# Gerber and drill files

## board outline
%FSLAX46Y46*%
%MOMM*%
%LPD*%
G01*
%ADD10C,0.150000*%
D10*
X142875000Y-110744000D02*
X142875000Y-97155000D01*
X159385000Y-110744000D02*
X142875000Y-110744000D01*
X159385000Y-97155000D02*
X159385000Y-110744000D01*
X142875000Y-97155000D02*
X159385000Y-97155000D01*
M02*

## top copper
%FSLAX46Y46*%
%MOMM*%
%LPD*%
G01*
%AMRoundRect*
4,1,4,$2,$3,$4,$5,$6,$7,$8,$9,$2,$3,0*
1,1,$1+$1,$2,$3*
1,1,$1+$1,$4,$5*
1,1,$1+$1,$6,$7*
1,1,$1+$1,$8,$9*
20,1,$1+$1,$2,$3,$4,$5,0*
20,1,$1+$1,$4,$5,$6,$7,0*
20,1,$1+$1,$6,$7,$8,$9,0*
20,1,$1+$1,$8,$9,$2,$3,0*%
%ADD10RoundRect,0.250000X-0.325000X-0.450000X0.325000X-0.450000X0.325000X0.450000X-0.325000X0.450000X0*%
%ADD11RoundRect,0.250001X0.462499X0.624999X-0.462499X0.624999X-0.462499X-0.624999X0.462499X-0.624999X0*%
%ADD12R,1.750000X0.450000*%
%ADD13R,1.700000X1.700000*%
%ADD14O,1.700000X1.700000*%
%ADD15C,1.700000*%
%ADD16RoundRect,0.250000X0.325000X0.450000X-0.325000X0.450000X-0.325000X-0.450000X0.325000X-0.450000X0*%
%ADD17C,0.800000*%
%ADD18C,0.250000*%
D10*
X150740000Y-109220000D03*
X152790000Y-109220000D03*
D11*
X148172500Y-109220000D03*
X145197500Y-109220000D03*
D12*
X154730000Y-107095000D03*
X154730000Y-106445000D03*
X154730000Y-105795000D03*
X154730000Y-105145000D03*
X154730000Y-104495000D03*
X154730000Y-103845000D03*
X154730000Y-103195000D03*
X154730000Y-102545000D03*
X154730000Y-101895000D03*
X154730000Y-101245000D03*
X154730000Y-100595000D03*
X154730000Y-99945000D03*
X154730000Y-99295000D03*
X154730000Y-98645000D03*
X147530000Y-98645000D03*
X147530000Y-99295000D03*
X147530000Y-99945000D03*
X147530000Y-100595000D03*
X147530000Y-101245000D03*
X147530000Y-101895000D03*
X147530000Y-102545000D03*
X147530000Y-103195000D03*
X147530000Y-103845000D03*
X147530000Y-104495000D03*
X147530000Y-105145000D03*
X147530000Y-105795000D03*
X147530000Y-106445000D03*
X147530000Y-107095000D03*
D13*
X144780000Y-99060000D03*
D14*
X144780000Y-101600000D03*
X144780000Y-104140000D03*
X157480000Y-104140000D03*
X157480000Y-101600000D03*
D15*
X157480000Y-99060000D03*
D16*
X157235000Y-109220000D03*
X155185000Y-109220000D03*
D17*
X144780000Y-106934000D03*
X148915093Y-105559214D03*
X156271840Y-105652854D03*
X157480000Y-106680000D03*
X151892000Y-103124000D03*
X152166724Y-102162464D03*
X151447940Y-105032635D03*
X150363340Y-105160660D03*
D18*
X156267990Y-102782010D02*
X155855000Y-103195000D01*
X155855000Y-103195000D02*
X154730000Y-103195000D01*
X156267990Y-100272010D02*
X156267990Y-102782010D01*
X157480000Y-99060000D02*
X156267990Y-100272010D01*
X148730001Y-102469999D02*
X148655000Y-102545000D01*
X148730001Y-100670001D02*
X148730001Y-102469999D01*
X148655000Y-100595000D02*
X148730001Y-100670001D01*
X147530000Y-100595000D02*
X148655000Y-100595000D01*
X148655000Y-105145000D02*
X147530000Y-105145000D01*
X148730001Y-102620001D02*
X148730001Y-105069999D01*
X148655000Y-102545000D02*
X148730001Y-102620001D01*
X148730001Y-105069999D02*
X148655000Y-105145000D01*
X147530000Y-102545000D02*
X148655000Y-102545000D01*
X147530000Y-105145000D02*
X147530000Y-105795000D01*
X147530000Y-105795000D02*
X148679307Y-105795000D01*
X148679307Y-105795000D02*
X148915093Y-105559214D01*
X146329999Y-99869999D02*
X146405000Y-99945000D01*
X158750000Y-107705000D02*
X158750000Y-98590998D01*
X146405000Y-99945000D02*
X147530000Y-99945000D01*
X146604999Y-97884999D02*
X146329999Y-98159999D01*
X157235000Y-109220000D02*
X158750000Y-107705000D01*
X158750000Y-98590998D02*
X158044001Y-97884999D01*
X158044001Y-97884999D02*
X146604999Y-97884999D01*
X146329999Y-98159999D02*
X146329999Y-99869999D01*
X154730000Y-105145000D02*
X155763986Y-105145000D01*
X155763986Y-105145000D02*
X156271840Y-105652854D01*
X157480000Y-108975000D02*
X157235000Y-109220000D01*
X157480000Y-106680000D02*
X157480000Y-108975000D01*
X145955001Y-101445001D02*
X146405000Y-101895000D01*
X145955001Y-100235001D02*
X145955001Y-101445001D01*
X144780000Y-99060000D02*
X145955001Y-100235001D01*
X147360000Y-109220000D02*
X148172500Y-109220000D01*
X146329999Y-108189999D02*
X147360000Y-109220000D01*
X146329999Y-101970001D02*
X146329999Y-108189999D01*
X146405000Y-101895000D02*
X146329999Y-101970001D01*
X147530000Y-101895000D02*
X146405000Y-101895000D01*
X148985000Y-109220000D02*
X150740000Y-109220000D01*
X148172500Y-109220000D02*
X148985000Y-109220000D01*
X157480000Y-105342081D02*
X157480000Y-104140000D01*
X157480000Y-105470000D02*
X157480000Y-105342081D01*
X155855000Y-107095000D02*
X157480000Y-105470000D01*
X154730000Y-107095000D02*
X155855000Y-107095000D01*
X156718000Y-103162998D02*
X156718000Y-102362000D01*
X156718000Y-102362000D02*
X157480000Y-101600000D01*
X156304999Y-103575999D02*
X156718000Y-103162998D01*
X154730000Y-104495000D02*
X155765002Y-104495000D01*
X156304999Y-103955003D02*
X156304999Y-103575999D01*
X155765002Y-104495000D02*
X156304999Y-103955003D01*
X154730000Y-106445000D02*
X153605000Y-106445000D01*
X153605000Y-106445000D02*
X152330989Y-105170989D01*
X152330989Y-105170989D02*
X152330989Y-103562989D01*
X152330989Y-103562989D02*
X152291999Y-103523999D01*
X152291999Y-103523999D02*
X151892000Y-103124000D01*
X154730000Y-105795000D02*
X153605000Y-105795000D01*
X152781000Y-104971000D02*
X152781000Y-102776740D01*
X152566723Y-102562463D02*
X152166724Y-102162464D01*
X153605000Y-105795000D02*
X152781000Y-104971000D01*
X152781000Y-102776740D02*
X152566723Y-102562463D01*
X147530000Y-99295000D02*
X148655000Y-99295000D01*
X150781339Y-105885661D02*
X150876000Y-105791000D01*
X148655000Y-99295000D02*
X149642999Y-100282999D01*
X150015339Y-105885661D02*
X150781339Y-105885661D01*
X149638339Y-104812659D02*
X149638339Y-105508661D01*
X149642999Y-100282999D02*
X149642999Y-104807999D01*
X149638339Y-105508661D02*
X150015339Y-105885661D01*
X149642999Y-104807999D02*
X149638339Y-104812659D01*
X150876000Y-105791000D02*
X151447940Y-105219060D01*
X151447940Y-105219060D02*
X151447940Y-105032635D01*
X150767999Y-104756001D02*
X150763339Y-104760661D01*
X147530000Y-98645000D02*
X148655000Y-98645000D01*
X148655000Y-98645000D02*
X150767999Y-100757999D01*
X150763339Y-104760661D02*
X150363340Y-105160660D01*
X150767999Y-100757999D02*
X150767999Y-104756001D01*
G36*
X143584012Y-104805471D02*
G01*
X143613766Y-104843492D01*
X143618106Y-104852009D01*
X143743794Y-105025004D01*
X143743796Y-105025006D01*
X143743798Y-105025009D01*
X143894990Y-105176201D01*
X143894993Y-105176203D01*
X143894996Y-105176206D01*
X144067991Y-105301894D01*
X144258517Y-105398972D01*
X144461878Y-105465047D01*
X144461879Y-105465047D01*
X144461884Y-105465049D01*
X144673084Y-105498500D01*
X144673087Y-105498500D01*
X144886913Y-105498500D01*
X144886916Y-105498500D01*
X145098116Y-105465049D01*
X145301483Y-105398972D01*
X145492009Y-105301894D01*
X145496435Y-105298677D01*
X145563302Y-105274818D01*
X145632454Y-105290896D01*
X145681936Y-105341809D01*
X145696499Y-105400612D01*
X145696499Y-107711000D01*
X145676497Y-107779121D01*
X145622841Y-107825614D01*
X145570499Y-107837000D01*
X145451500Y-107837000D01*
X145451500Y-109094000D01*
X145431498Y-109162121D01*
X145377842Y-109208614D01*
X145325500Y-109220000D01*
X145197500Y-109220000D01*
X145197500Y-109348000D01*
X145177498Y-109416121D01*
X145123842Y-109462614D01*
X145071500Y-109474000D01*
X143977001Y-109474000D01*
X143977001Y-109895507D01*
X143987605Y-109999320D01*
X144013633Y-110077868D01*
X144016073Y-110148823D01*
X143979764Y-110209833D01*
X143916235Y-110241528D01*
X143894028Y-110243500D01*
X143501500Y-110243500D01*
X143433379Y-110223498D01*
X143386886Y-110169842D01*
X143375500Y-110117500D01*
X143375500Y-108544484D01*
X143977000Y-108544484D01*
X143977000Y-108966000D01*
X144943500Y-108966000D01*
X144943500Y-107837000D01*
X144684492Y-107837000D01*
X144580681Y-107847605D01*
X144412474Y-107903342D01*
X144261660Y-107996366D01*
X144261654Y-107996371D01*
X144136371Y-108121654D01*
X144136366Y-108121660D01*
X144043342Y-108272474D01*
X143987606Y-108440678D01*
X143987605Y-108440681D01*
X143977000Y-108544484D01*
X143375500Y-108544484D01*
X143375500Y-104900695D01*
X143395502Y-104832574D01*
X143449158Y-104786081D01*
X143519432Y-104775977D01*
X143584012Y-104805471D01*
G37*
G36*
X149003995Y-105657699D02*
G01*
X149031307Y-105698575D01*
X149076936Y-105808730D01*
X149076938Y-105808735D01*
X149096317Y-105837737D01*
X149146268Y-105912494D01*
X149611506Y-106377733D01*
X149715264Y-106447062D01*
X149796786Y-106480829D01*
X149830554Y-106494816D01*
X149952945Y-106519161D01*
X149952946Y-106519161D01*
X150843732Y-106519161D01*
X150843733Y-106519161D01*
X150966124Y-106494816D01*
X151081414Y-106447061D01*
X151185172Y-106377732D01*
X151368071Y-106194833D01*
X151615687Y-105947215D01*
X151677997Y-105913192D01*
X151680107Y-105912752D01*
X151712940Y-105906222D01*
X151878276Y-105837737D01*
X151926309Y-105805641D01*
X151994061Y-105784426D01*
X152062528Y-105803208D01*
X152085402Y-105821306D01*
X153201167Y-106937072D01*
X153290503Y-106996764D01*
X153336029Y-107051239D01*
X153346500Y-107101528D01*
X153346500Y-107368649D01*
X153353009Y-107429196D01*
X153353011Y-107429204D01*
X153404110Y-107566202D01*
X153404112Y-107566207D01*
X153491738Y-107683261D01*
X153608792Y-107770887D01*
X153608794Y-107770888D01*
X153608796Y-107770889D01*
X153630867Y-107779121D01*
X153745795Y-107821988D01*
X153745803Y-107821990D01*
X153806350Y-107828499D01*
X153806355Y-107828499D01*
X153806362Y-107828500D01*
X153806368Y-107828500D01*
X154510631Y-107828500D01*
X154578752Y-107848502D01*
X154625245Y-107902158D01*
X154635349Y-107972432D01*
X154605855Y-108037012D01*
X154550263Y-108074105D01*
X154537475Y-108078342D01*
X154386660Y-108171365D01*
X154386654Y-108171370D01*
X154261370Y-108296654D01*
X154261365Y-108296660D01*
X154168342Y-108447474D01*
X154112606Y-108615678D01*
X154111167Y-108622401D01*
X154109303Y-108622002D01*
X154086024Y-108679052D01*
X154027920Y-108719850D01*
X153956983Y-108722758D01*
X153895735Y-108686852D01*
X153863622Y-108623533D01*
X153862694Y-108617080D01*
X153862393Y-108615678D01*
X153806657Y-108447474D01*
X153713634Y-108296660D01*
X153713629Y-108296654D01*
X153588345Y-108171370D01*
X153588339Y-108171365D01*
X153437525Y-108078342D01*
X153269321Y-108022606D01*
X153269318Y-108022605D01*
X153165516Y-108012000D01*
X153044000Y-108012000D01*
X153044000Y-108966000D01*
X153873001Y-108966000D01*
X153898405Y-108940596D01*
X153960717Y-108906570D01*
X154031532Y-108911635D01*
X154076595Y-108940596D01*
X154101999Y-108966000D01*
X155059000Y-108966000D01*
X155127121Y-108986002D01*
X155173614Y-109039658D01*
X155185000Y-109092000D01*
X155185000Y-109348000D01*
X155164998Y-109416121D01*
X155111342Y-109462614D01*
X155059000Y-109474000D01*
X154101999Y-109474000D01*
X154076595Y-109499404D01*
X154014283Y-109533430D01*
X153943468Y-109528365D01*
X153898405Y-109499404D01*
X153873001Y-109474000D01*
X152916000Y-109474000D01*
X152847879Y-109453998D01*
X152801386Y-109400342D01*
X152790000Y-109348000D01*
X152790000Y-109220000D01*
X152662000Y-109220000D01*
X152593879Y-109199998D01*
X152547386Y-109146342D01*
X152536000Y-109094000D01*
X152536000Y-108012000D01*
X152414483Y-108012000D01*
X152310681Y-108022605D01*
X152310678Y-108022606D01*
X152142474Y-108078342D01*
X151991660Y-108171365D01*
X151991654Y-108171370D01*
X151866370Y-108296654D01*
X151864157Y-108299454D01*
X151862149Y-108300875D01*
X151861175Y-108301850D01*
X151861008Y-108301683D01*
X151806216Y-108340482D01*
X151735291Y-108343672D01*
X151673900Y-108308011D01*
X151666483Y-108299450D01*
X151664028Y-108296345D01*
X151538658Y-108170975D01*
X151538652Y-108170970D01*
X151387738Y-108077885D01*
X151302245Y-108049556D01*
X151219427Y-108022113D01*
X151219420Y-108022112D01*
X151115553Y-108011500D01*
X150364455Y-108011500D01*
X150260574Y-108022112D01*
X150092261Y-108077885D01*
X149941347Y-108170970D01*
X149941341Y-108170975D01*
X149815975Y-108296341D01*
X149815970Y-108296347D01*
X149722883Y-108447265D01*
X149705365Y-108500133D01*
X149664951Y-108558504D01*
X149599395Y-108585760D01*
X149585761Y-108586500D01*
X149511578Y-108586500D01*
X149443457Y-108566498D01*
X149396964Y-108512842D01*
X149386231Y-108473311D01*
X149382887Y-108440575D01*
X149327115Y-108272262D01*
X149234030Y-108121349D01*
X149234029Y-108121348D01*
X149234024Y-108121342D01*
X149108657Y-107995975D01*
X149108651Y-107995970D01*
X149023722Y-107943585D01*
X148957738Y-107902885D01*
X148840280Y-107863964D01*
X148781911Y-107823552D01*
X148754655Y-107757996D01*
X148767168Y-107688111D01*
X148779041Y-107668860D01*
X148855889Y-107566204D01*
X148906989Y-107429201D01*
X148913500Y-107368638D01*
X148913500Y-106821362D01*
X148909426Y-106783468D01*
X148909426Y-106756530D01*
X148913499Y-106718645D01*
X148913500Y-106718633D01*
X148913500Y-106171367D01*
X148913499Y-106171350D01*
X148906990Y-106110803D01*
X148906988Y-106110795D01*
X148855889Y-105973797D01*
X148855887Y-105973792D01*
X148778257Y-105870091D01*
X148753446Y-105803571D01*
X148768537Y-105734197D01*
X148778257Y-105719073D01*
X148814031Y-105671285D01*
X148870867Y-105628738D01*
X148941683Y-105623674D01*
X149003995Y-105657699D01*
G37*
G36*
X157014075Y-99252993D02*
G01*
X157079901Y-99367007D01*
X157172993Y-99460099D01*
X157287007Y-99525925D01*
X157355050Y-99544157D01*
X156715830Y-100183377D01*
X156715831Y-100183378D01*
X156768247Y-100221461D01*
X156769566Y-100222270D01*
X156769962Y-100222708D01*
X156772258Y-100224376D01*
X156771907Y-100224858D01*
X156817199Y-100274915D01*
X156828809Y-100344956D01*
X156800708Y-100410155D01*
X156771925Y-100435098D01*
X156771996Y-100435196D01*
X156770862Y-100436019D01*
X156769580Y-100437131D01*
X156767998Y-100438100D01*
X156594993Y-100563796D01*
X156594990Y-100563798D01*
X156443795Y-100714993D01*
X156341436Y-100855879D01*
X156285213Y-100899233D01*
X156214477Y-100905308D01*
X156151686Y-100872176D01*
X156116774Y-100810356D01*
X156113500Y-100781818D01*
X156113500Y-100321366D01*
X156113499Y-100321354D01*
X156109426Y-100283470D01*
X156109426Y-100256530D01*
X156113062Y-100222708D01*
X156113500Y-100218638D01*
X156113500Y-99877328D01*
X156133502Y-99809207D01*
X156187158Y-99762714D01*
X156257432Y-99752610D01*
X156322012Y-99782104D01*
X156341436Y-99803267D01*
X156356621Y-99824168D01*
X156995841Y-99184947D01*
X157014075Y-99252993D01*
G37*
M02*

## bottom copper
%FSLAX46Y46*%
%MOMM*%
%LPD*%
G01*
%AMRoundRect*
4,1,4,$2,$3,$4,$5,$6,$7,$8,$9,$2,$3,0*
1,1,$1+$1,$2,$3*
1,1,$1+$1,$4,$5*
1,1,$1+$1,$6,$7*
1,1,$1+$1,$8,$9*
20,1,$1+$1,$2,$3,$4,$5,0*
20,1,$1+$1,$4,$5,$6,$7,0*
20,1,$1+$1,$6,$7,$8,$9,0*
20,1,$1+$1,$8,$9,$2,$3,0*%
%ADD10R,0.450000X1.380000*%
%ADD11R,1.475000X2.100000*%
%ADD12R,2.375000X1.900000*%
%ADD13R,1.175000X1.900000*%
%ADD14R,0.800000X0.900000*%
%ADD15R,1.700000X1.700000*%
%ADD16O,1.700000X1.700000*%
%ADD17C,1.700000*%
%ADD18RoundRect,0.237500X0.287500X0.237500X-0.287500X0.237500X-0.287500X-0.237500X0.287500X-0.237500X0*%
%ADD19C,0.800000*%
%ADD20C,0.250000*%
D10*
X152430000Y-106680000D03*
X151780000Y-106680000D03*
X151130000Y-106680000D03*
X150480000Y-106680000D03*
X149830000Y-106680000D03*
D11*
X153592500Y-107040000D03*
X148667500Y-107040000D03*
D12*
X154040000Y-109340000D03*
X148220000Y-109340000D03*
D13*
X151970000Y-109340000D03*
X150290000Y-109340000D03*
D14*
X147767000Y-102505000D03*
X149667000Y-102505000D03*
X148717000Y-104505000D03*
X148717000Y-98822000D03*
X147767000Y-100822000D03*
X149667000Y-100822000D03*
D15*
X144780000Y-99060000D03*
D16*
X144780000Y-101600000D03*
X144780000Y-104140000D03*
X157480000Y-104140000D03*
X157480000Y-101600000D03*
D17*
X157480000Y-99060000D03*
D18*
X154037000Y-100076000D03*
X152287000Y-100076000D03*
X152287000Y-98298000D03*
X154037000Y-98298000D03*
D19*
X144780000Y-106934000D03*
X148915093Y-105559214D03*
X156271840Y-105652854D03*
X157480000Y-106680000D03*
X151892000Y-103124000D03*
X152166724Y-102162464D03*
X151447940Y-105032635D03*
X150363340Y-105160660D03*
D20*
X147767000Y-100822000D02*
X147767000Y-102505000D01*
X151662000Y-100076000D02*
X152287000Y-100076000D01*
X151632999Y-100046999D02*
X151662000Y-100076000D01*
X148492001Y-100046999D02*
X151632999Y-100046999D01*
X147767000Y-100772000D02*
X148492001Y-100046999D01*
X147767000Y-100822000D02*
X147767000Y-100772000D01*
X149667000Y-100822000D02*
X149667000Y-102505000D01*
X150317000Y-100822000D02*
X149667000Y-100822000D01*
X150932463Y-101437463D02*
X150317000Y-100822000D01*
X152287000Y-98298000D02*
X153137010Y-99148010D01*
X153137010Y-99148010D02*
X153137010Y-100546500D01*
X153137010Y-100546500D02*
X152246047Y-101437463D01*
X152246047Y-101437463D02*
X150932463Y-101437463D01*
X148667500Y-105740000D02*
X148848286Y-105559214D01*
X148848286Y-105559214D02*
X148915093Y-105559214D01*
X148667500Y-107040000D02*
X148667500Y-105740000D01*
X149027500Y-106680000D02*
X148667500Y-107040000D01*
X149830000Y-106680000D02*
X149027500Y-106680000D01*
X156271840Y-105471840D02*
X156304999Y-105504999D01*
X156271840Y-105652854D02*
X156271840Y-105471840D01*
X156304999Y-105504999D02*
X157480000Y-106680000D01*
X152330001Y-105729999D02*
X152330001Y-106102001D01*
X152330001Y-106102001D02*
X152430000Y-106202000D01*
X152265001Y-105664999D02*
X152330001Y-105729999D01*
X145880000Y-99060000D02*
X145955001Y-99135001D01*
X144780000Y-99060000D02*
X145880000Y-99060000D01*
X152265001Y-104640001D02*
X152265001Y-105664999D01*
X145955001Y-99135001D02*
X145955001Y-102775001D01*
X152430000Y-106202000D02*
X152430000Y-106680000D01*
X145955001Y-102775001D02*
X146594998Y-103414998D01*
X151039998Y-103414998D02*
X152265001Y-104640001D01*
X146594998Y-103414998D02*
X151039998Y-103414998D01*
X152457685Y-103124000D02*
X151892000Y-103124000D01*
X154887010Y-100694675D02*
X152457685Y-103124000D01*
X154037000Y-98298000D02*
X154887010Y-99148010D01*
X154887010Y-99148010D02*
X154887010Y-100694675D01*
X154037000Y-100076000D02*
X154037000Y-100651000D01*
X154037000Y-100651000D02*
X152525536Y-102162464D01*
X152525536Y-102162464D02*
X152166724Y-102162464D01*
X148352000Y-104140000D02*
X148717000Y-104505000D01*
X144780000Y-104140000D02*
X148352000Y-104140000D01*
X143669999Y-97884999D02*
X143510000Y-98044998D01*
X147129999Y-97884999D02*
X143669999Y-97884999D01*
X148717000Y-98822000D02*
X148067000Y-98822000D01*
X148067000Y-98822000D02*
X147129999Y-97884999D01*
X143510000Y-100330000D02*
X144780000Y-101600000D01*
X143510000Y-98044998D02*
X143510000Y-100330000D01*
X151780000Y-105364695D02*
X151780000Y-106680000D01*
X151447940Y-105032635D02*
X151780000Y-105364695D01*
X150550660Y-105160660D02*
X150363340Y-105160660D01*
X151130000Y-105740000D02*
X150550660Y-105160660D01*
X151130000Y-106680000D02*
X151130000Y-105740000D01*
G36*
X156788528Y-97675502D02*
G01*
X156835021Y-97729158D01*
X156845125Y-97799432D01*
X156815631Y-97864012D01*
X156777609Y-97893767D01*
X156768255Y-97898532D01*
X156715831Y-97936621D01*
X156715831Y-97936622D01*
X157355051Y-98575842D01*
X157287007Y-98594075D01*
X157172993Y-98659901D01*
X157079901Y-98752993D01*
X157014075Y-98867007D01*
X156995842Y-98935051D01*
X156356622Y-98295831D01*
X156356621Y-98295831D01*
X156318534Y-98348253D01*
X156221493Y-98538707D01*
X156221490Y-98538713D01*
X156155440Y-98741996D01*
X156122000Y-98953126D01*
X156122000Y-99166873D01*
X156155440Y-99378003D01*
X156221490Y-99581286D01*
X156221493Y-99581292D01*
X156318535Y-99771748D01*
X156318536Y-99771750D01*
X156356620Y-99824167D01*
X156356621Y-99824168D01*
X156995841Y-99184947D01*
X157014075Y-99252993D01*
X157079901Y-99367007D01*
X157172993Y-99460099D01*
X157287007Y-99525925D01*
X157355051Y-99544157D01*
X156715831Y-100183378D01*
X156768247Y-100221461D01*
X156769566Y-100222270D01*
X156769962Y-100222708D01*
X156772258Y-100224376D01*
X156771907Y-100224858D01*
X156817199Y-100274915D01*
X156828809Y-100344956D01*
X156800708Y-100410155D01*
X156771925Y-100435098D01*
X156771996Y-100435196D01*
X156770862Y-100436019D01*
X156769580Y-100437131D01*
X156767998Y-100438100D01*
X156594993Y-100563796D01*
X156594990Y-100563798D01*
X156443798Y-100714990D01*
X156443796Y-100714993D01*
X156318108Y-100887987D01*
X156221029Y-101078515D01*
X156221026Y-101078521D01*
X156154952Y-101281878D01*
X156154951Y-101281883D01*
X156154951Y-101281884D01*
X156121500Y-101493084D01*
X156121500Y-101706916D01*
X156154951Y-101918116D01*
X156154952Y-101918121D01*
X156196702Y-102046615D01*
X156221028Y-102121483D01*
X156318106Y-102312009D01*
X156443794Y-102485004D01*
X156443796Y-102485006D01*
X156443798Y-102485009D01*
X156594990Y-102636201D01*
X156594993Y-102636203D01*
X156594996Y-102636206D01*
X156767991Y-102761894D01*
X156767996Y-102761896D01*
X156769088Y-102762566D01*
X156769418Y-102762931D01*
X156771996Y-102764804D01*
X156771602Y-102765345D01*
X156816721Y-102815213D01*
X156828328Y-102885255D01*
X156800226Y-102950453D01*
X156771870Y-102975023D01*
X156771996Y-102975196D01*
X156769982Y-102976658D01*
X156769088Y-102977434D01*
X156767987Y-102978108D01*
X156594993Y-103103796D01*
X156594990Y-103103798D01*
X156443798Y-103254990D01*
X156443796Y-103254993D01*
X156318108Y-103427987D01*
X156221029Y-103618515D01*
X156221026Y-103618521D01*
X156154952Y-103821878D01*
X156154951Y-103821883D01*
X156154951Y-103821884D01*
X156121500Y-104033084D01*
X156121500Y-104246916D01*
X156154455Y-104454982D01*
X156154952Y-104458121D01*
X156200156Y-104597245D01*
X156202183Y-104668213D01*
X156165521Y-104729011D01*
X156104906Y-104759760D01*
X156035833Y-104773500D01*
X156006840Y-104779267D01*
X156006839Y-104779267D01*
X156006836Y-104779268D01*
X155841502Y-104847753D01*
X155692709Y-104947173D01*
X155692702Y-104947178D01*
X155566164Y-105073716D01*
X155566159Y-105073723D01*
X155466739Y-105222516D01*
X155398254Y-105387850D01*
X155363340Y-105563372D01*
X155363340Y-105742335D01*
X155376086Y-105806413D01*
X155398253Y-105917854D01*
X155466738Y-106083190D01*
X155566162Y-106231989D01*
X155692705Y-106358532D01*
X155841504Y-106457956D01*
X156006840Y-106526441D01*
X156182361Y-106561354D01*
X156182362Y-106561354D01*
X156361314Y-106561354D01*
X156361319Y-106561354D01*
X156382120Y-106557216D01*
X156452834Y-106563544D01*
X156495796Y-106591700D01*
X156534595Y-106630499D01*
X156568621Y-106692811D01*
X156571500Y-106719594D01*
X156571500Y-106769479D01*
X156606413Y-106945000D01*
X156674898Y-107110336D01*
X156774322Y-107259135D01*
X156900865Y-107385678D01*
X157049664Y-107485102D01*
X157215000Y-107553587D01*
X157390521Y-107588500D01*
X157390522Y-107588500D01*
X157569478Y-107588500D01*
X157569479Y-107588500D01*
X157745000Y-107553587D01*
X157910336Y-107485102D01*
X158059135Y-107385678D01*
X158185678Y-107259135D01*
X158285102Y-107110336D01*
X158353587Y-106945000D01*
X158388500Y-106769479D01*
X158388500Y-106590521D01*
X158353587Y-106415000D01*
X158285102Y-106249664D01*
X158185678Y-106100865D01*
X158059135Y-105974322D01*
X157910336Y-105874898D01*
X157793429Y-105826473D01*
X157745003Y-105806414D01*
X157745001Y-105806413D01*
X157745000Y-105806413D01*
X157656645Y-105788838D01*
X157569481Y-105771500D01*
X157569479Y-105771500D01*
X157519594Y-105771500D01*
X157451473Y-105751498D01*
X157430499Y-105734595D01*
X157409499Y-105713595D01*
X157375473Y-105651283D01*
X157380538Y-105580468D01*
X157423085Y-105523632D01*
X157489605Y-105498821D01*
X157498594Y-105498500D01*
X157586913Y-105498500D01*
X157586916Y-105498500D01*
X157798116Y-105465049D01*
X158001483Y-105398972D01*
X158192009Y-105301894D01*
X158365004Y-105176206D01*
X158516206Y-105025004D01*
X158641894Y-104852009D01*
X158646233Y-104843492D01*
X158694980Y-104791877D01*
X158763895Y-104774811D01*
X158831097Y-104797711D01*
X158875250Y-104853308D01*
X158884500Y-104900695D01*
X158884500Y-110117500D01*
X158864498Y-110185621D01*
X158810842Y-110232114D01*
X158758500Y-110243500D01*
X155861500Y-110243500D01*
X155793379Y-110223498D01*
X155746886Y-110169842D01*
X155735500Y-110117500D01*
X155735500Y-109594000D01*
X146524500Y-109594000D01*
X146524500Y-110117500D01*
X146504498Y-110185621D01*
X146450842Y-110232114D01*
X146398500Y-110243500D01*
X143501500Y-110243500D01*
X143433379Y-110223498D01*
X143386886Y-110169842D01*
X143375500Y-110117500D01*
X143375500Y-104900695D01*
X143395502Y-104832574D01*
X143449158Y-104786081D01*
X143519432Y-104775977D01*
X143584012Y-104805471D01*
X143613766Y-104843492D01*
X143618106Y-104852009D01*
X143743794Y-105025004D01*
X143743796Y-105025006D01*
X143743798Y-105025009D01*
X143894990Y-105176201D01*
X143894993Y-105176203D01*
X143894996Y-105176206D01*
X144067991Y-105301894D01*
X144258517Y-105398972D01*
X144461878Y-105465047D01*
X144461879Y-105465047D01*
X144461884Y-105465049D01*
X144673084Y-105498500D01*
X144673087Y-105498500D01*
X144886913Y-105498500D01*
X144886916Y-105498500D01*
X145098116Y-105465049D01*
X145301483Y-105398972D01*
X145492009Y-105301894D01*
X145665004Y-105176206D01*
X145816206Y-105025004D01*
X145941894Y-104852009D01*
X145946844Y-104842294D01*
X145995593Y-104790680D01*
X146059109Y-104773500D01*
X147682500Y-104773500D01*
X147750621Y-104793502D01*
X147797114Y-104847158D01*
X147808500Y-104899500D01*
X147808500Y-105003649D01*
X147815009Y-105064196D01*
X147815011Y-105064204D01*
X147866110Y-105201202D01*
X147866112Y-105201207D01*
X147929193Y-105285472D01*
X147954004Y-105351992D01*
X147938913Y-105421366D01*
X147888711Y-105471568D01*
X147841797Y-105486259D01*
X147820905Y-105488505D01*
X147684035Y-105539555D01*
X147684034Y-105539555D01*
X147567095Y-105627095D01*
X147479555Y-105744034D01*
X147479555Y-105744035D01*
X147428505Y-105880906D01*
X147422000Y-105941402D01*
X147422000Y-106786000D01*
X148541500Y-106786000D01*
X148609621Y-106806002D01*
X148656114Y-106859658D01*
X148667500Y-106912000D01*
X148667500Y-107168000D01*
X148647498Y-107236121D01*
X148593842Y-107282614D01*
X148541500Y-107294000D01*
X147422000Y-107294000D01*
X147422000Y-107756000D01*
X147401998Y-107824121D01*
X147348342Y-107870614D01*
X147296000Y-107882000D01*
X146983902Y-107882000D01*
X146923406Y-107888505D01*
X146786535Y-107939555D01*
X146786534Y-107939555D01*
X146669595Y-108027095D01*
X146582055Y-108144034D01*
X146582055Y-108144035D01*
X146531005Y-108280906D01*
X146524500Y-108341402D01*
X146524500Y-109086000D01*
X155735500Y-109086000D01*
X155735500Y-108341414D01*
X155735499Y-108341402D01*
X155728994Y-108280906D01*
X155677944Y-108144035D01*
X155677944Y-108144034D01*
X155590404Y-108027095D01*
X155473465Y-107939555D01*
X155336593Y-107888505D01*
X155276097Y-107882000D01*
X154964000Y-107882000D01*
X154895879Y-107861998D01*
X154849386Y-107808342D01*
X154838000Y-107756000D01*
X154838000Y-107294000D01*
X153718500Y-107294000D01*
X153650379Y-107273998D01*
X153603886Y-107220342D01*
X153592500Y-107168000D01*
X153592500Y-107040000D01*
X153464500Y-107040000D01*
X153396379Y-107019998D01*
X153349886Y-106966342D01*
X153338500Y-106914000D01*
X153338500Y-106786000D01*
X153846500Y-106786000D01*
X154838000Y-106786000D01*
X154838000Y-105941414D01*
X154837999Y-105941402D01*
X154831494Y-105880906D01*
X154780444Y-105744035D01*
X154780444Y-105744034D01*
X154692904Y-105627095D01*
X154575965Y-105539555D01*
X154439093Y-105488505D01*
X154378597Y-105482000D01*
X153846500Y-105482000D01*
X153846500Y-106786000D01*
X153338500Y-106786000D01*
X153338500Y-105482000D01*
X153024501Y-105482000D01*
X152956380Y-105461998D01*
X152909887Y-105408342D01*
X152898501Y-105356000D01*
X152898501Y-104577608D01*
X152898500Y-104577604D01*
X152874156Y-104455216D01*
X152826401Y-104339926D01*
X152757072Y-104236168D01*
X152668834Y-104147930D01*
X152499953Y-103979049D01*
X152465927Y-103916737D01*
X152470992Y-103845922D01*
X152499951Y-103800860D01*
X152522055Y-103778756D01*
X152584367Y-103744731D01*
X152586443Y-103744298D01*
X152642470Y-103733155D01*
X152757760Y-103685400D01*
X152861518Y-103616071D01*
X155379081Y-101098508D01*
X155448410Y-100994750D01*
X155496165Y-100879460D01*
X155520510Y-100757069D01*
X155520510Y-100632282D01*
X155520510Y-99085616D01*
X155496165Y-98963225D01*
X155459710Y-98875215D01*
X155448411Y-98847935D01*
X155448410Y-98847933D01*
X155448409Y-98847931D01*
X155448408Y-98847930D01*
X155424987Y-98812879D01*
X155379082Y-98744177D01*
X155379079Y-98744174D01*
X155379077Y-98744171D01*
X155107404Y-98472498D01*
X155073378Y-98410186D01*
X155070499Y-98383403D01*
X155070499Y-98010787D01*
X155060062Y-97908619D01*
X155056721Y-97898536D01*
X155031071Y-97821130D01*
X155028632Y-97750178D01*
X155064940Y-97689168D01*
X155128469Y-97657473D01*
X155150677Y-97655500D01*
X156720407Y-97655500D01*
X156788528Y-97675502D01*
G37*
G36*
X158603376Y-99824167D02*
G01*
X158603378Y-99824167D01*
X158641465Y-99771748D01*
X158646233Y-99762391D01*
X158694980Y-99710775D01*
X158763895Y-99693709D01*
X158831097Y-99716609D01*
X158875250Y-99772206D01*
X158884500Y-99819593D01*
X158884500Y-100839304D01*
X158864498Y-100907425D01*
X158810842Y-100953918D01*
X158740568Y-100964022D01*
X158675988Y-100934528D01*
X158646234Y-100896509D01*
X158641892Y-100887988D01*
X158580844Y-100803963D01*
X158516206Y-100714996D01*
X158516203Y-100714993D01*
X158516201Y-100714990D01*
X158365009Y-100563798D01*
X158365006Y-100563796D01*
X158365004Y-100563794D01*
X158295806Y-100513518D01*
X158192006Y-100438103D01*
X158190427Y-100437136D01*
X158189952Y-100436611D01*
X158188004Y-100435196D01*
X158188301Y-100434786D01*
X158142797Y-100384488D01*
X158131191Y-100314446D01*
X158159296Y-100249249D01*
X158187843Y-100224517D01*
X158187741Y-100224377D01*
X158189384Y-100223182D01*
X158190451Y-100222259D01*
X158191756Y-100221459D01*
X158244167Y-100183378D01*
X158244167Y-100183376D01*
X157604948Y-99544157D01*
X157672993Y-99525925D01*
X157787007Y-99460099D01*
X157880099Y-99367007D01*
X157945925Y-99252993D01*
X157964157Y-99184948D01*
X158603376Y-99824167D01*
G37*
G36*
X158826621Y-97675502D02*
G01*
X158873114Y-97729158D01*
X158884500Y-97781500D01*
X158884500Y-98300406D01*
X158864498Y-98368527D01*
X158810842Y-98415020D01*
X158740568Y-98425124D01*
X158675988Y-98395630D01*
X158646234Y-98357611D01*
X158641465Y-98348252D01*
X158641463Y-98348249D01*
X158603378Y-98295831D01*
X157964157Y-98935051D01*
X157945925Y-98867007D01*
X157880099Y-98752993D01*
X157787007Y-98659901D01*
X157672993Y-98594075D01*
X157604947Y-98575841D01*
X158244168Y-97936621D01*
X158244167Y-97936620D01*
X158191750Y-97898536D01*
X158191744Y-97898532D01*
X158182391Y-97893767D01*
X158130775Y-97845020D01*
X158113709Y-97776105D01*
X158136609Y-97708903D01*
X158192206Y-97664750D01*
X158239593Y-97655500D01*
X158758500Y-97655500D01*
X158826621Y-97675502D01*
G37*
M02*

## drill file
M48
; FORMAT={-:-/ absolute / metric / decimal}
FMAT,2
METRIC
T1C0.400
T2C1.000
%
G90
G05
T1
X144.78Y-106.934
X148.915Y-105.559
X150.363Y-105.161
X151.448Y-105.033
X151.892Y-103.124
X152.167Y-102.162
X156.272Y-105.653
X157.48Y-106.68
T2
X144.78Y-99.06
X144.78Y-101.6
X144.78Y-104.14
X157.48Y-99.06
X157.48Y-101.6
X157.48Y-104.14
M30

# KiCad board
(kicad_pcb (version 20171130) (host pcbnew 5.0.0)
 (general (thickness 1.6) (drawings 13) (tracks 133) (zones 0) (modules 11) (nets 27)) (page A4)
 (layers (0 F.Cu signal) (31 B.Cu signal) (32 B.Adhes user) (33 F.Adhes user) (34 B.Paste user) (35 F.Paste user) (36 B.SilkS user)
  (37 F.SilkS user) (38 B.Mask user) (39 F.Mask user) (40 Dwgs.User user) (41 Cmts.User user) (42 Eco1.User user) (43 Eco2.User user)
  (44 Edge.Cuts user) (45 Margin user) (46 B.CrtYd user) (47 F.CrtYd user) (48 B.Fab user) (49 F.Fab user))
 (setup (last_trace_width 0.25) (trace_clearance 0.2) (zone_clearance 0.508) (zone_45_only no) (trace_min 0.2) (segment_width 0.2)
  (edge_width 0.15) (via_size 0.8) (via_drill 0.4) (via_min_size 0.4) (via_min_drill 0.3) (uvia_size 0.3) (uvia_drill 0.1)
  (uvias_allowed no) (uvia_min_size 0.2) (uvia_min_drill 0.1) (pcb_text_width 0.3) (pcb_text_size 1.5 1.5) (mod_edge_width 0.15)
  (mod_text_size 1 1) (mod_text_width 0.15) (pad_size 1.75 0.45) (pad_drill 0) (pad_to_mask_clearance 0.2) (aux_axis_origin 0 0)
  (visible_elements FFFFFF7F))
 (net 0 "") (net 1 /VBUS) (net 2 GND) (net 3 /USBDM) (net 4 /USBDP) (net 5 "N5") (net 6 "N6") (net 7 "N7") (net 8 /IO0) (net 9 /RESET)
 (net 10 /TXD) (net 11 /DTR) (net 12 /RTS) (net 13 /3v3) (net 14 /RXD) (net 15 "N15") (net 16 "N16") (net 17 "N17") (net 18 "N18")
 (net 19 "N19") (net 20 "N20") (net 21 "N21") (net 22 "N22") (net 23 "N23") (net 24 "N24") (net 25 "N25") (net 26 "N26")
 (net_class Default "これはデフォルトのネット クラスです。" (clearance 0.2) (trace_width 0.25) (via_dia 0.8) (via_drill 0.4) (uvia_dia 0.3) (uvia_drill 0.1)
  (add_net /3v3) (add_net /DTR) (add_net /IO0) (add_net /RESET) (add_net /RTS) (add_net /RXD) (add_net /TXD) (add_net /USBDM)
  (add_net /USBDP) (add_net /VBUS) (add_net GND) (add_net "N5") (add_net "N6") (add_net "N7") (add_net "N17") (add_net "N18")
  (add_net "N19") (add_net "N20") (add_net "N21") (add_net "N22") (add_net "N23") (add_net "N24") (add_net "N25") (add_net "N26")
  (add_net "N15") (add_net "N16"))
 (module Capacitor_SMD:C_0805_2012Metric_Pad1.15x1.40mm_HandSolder (layer F.Cu) (at 151.765 109.22)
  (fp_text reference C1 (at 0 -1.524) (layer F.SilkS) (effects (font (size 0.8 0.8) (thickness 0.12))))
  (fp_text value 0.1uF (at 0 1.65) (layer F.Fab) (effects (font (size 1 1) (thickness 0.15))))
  (pad 1 smd roundrect (at -1.025 0) (size 1.15 1.4) (layers F.Cu F.Paste F.Mask) (roundrect_rratio 0.217391) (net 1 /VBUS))
  (pad 2 smd roundrect (at 1.025 0) (size 1.15 1.4) (layers F.Cu F.Paste F.Mask) (roundrect_rratio 0.217391) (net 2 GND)))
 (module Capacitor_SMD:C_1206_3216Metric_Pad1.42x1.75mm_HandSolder (layer F.Cu) (at 146.685 109.22 180)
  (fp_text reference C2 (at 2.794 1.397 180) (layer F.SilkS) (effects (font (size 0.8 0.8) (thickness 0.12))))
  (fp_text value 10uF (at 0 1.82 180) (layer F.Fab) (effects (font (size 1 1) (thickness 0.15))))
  (pad 1 smd roundrect (at -1.4875 0 180) (size 1.425 1.75) (layers F.Cu F.Paste F.Mask) (roundrect_rratio 0.175439) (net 1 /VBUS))
  (pad 2 smd roundrect (at 1.4875 0 180) (size 1.425 1.75) (layers F.Cu F.Paste F.Mask) (roundrect_rratio 0.175439) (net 2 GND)))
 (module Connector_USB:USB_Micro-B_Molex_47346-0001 (layer B.Cu) (at 151.13 108.14 180)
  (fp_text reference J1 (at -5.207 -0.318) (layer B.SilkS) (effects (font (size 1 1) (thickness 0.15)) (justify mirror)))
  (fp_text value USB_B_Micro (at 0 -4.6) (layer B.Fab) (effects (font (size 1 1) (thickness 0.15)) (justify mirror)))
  (pad 1 smd rect (at -1.3 1.46 180) (size 0.45 1.38) (layers B.Cu B.Paste B.Mask) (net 1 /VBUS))
  (pad 2 smd rect (at -0.65 1.46 180) (size 0.45 1.38) (layers B.Cu B.Paste B.Mask) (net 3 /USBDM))
  (pad 3 smd rect (at 0 1.46 180) (size 0.45 1.38) (layers B.Cu B.Paste B.Mask) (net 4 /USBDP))
  (pad 4 smd rect (at 0.65 1.46 180) (size 0.45 1.38) (layers B.Cu B.Paste B.Mask) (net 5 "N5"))
  (pad 5 smd rect (at 1.3 1.46 180) (size 0.45 1.38) (layers B.Cu B.Paste B.Mask) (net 2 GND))
  (pad 6 smd rect (at -2.4625 1.1 180) (size 1.475 2.1) (layers B.Cu B.Paste B.Mask) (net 2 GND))
  (pad 6 smd rect (at 2.4625 1.1 180) (size 1.475 2.1) (layers B.Cu B.Paste B.Mask) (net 2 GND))
  (pad 6 smd rect (at -2.91 -1.2 180) (size 2.375 1.9) (layers B.Cu B.Paste B.Mask) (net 2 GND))
  (pad 6 smd rect (at 2.91 -1.2 180) (size 2.375 1.9) (layers B.Cu B.Paste B.Mask) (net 2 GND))
  (pad 6 smd rect (at -0.84 -1.2 180) (size 1.175 1.9) (layers B.Cu B.Paste B.Mask) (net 2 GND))
  (pad 6 smd rect (at 0.84 -1.2 180) (size 1.175 1.9) (layers B.Cu B.Paste B.Mask) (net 2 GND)))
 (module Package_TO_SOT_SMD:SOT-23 (layer B.Cu) (at 148.717 103.505 270)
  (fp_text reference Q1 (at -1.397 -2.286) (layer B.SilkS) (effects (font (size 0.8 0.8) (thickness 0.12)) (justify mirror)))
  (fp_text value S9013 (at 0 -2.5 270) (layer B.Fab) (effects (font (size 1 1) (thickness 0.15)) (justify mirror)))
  (pad 1 smd rect (at -1 0.95 270) (size 0.9 0.8) (layers B.Cu B.Paste B.Mask) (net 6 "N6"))
  (pad 2 smd rect (at -1 -0.95 270) (size 0.9 0.8) (layers B.Cu B.Paste B.Mask) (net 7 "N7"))
  (pad 3 smd rect (at 1 0 270) (size 0.9 0.8) (layers B.Cu B.Paste B.Mask) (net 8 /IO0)))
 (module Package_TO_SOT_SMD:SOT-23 (layer B.Cu) (at 148.717 99.822 90)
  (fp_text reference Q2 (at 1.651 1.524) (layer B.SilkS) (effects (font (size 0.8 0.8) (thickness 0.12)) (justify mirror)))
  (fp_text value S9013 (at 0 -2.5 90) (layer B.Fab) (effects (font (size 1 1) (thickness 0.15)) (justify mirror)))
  (pad 3 smd rect (at 1 0 90) (size 0.9 0.8) (layers B.Cu B.Paste B.Mask) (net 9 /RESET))
  (pad 2 smd rect (at -1 -0.95 90) (size 0.9 0.8) (layers B.Cu B.Paste B.Mask) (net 6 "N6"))
  (pad 1 smd rect (at -1 0.95 90) (size 0.9 0.8) (layers B.Cu B.Paste B.Mask) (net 7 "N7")))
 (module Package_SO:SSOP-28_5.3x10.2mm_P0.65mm (layer F.Cu) (at 151.13 102.87 180)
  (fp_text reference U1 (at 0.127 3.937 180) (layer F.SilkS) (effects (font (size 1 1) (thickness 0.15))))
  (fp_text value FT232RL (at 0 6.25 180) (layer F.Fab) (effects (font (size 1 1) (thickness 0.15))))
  (pad 1 smd rect (at -3.6 -4.225 180) (size 1.75 0.45) (layers F.Cu F.Paste F.Mask) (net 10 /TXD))
  (pad 2 smd rect (at -3.6 -3.575 180) (size 1.75 0.45) (layers F.Cu F.Paste F.Mask) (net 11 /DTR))
  (pad 3 smd rect (at -3.6 -2.925 180) (size 1.75 0.45) (layers F.Cu F.Paste F.Mask) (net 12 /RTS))
  (pad 4 smd rect (at -3.6 -2.275 180) (size 1.75 0.45) (layers F.Cu F.Paste F.Mask) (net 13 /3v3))
  (pad 5 smd rect (at -3.6 -1.625 180) (size 1.75 0.45) (layers F.Cu F.Paste F.Mask) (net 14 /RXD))
  (pad 6 smd rect (at -3.6 -0.975 180) (size 1.75 0.45) (layers F.Cu F.Paste F.Mask) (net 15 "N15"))
  (pad 7 smd rect (at -3.6 -0.325 180) (size 1.75 0.45) (layers F.Cu F.Paste F.Mask) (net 2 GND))
  (pad 8 smd rect (at -3.6 0.325 180) (size 1.75 0.45) (layers F.Cu F.Paste F.Mask))
  (pad 9 smd rect (at -3.6 0.975 180) (size 1.75 0.45) (layers F.Cu F.Paste F.Mask) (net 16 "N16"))
  (pad 10 smd rect (at -3.6 1.625 180) (size 1.75 0.45) (layers F.Cu F.Paste F.Mask) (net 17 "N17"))
  (pad 11 smd rect (at -3.6 2.275 180) (size 1.75 0.45) (layers F.Cu F.Paste F.Mask) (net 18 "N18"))
  (pad 12 smd rect (at -3.6 2.925 180) (size 1.75 0.45) (layers F.Cu F.Paste F.Mask) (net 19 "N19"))
  (pad 13 smd rect (at -3.6 3.575 180) (size 1.75 0.45) (layers F.Cu F.Paste F.Mask) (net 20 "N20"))
  (pad 14 smd rect (at -3.6 4.225 180) (size 1.75 0.45) (layers F.Cu F.Paste F.Mask) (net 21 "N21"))
  (pad 15 smd rect (at 3.6 4.225 180) (size 1.75 0.45) (layers F.Cu F.Paste F.Mask) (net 4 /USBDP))
  (pad 16 smd rect (at 3.6 3.575 180) (size 1.75 0.45) (layers F.Cu F.Paste F.Mask) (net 3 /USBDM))
  (pad 17 smd rect (at 3.6 2.925 180) (size 1.75 0.45) (layers F.Cu F.Paste F.Mask) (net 13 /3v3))
  (pad 18 smd rect (at 3.6 2.275 180) (size 1.75 0.45) (layers F.Cu F.Paste F.Mask) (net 2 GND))
  (pad 19 smd rect (at 3.6 1.625 180) (size 1.75 0.45) (layers F.Cu F.Paste F.Mask) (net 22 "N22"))
  (pad 20 smd rect (at 3.6 0.975 180) (size 1.75 0.45) (layers F.Cu F.Paste F.Mask) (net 1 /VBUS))
  (pad 21 smd rect (at 3.6 0.325 180) (size 1.75 0.45) (layers F.Cu F.Paste F.Mask) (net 2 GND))
  (pad 22 smd rect (at 3.6 -0.325 180) (size 1.75 0.45) (layers F.Cu F.Paste F.Mask) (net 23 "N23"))
  (pad 23 smd rect (at 3.6 -0.975 180) (size 1.75 0.45) (layers F.Cu F.Paste F.Mask) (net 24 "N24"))
  (pad 24 smd rect (at 3.6 -1.625 180) (size 1.75 0.45) (layers F.Cu F.Paste F.Mask))
  (pad 25 smd rect (at 3.6 -2.275 180) (size 1.75 0.45) (layers F.Cu F.Paste F.Mask) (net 2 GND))
  (pad 26 smd rect (at 3.6 -2.925 180) (size 1.75 0.45) (layers F.Cu F.Paste F.Mask) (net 2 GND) (zone_connect 2))
  (pad 27 smd rect (at 3.6 -3.575 180) (size 1.75 0.45) (layers F.Cu F.Paste F.Mask) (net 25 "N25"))
  (pad 28 smd rect (at 3.6 -4.225 180) (size 1.75 0.45) (layers F.Cu F.Paste F.Mask) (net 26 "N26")))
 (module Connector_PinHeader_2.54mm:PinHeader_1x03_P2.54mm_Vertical (layer B.Cu) (at 144.78 99.06 180)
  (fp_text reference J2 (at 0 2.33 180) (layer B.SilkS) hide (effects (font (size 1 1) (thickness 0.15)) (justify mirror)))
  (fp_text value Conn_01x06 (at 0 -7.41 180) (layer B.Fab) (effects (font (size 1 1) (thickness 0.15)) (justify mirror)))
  (pad 1 thru_hole rect (at 0 0 180) (size 1.7 1.7) (drill 1) (layers *.Cu *.Mask) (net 1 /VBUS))
  (pad 2 thru_hole oval (at 0 -2.54 180) (size 1.7 1.7) (drill 1) (layers *.Cu *.Mask) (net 9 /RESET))
  (pad 3 thru_hole oval (at 0 -5.08 180) (size 1.7 1.7) (drill 1) (layers *.Cu *.Mask) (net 8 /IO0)))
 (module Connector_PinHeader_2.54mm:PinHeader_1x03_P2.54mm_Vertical (layer B.Cu) (at 157.48 99.06 180)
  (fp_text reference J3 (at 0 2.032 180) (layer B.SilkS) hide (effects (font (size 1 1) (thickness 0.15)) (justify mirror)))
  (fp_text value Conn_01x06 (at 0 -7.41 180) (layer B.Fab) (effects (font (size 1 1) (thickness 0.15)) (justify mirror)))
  (pad 3 thru_hole oval (at 0 -5.08 180) (size 1.7 1.7) (drill 1) (layers *.Cu *.Mask) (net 10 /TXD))
  (pad 2 thru_hole oval (at 0 -2.54 180) (size 1.7 1.7) (drill 1) (layers *.Cu *.Mask) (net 14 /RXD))
  (pad 1 thru_hole circle (at 0 0 180) (size 1.7 1.7) (drill 1) (layers *.Cu *.Mask) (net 2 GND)))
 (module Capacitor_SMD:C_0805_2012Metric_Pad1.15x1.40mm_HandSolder (layer F.Cu) (at 156.21 109.22 180)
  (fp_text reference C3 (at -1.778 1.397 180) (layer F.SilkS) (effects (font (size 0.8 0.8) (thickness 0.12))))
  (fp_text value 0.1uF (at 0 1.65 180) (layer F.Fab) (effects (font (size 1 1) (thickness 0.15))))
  (pad 1 smd roundrect (at -1.025 0 180) (size 1.15 1.4) (layers F.Cu F.Paste F.Mask) (roundrect_rratio 0.217391) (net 13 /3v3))
  (pad 2 smd roundrect (at 1.025 0 180) (size 1.15 1.4) (layers F.Cu F.Paste F.Mask) (roundrect_rratio 0.217391) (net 2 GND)))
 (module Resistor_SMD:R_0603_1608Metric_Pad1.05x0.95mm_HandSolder (layer B.Cu) (at 153.162 100.076 180)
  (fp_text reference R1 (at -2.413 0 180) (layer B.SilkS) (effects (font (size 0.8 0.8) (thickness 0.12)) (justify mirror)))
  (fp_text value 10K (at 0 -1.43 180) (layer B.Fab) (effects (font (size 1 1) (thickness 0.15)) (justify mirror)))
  (pad 1 smd roundrect (at -0.875 0 180) (size 1.05 0.95) (layers B.Cu B.Paste B.Mask) (roundrect_rratio 0.25) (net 12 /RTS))
  (pad 2 smd roundrect (at 0.875 0 180) (size 1.05 0.95) (layers B.Cu B.Paste B.Mask) (roundrect_rratio 0.25) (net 6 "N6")))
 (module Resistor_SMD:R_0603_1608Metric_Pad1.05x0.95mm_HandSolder (layer B.Cu) (at 153.162 98.298 180)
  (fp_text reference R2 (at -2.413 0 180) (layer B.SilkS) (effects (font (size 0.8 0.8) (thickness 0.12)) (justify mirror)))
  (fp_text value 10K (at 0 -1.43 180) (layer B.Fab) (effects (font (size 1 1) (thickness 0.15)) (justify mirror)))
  (pad 2 smd roundrect (at 0.875 0 180) (size 1.05 0.95) (layers B.Cu B.Paste B.Mask) (roundrect_rratio 0.25) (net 7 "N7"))
  (pad 1 smd roundrect (at -0.875 0 180) (size 1.05 0.95) (layers B.Cu B.Paste B.Mask) (roundrect_rratio 0.25) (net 11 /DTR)))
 (gr_line (start 142.875 110.744) (end 142.875 97.155) (layer Edge.Cuts) (width 0.15))
 (gr_line (start 159.385 110.744) (end 142.875 110.744) (layer Edge.Cuts) (width 0.15))
 (gr_line (start 159.385 97.155) (end 159.385 110.744) (layer Edge.Cuts) (width 0.15))
 (gr_line (start 142.875 97.155) (end 159.385 97.155) (layer Edge.Cuts) (width 0.15))
 (segment (start 147.767 100.822) (end 147.767 102.505) (width 0.25) (layer B.Cu) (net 6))
 (segment (start 151.662 100.076) (end 152.287 100.076) (width 0.25) (layer B.Cu) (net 6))
 (segment (start 151.632999 100.046999) (end 151.662 100.076) (width 0.25) (layer B.Cu) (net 6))
 (segment (start 148.492001 100.046999) (end 151.632999 100.046999) (width 0.25) (layer B.Cu) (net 6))
 (segment (start 147.767 100.772) (end 148.492001 100.046999) (width 0.25) (layer B.Cu) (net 6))
 (segment (start 147.767 100.822) (end 147.767 100.772) (width 0.25) (layer B.Cu) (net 6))
 (segment (start 149.667 100.822) (end 149.667 102.505) (width 0.25) (layer B.Cu) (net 7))
 (segment (start 150.317 100.822) (end 149.667 100.822) (width 0.25) (layer B.Cu) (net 7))
 (segment (start 150.932463 101.437463) (end 150.317 100.822) (width 0.25) (layer B.Cu) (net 7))
 (segment (start 152.287 98.298) (end 153.13701 99.14801) (width 0.25) (layer B.Cu) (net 7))
 (segment (start 153.13701 99.14801) (end 153.13701 100.5465) (width 0.25) (layer B.Cu) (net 7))
 (segment (start 153.13701 100.5465) (end 152.246047 101.437463) (width 0.25) (layer B.Cu) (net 7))
 (segment (start 152.246047 101.437463) (end 150.932463 101.437463) (width 0.25) (layer B.Cu) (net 7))
 (segment (start 156.26799 102.78201) (end 155.855 103.195) (width 0.25) (layer F.Cu) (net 2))
 (segment (start 155.855 103.195) (end 154.73 103.195) (width 0.25) (layer F.Cu) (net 2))
 (segment (start 156.26799 100.27201) (end 156.26799 102.78201) (width 0.25) (layer F.Cu) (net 2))
 (segment (start 157.48 99.06) (end 156.26799 100.27201) (width 0.25) (layer F.Cu) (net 2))
 (segment (start 148.730001 102.469999) (end 148.655 102.545) (width 0.25) (layer F.Cu) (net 2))
 (segment (start 148.730001 100.670001) (end 148.730001 102.469999) (width 0.25) (layer F.Cu) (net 2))
 (segment (start 148.655 100.595) (end 148.730001 100.670001) (width 0.25) (layer F.Cu) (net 2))
 (segment (start 147.53 100.595) (end 148.655 100.595) (width 0.25) (layer F.Cu) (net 2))
 (segment (start 148.655 105.145) (end 147.53 105.145) (width 0.25) (layer F.Cu) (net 2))
 (segment (start 148.730001 102.620001) (end 148.730001 105.069999) (width 0.25) (layer F.Cu) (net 2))
 (segment (start 148.655 102.545) (end 148.730001 102.620001) (width 0.25) (layer F.Cu) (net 2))
 (segment (start 148.730001 105.069999) (end 148.655 105.145) (width 0.25) (layer F.Cu) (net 2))
 (segment (start 147.53 102.545) (end 148.655 102.545) (width 0.25) (layer F.Cu) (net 2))
 (segment (start 147.53 105.145) (end 147.53 105.795) (width 0.25) (layer F.Cu) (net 2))
 (segment (start 148.6675 105.74) (end 148.848286 105.559214) (width 0.25) (layer B.Cu) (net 2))
 (segment (start 147.53 105.795) (end 148.679307 105.795) (width 0.25) (layer F.Cu) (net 2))
 (segment (start 148.848286 105.559214) (end 148.915093 105.559214) (width 0.25) (layer B.Cu) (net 2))
 (segment (start 148.679307 105.795) (end 148.915093 105.559214) (width 0.25) (layer F.Cu) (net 2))
 (segment (start 148.6675 107.04) (end 148.6675 105.74) (width 0.25) (layer B.Cu) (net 2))
 (segment (start 149.0275 106.68) (end 148.6675 107.04) (width 0.25) (layer B.Cu) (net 2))
 (segment (start 149.83 106.68) (end 149.0275 106.68) (width 0.25) (layer B.Cu) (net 2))
 (via (at 144.78 106.934) (size 0.8) (drill 0.4) (layers F.Cu B.Cu) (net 2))
 (via (at 148.915093 105.559214) (size 0.8) (drill 0.4) (layers F.Cu B.Cu) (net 2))
 (segment (start 146.329999 99.869999) (end 146.405 99.945) (width 0.25) (layer F.Cu) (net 13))
 (segment (start 158.75 107.705) (end 158.75 98.590998) (width 0.25) (layer F.Cu) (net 13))
 (segment (start 146.405 99.945) (end 147.53 99.945) (width 0.25) (layer F.Cu) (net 13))
 (segment (start 146.604999 97.884999) (end 146.329999 98.159999) (width 0.25) (layer F.Cu) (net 13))
 (segment (start 157.235 109.22) (end 158.75 107.705) (width 0.25) (layer F.Cu) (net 13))
 (segment (start 158.75 98.590998) (end 158.044001 97.884999) (width 0.25) (layer F.Cu) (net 13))
 (segment (start 158.044001 97.884999) (end 146.604999 97.884999) (width 0.25) (layer F.Cu) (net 13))
 (segment (start 146.329999 98.159999) (end 146.329999 99.869999) (width 0.25) (layer F.Cu) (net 13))
 (via (at 156.27184 105.652854) (size 0.8) (drill 0.4) (layers F.Cu B.Cu) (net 13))
 (segment (start 154.73 105.145) (end 155.763986 105.145) (width 0.25) (layer F.Cu) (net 13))
 (segment (start 155.763986 105.145) (end 156.27184 105.652854) (width 0.25) (layer F.Cu) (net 13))
 (segment (start 156.27184 105.47184) (end 156.304999 105.504999) (width 0.25) (layer B.Cu) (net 13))
 (segment (start 156.27184 105.652854) (end 156.27184 105.47184) (width 0.25) (layer B.Cu) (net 13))
 (via (at 157.48 106.68) (size 0.8) (drill 0.4) (layers F.Cu B.Cu) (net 13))
 (segment (start 156.304999 105.504999) (end 157.48 106.68) (width 0.25) (layer B.Cu) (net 13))
 (segment (start 157.48 108.975) (end 157.235 109.22) (width 0.25) (layer F.Cu) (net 13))
 (segment (start 157.48 106.68) (end 157.48 108.975) (width 0.25) (layer F.Cu) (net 13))
 (segment (start 145.955001 101.445001) (end 146.405 101.895) (width 0.25) (layer F.Cu) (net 1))
 (segment (start 145.955001 100.235001) (end 145.955001 101.445001) (width 0.25) (layer F.Cu) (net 1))
 (segment (start 144.78 99.06) (end 145.955001 100.235001) (width 0.25) (layer F.Cu) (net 1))
 (segment (start 147.36 109.22) (end 148.1725 109.22) (width 0.25) (layer F.Cu) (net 1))
 (segment (start 146.329999 108.189999) (end 147.36 109.22) (width 0.25) (layer F.Cu) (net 1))
 (segment (start 146.329999 101.970001) (end 146.329999 108.189999) (width 0.25) (layer F.Cu) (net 1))
 (segment (start 146.405 101.895) (end 146.329999 101.970001) (width 0.25) (layer F.Cu) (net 1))
 (segment (start 147.53 101.895) (end 146.405 101.895) (width 0.25) (layer F.Cu) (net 1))
 (segment (start 148.985 109.22) (end 150.74 109.22) (width 0.25) (layer F.Cu) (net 1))
 (segment (start 148.1725 109.22) (end 148.985 109.22) (width 0.25) (layer F.Cu) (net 1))
 (segment (start 152.330001 105.729999) (end 152.330001 106.102001) (width 0.25) (layer B.Cu) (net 1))
 (segment (start 152.330001 106.102001) (end 152.43 106.202) (width 0.25) (layer B.Cu) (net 1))
 (segment (start 152.265001 105.664999) (end 152.330001 105.729999) (width 0.25) (layer B.Cu) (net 1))
 (segment (start 145.88 99.06) (end 145.955001 99.135001) (width 0.25) (layer B.Cu) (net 1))
 (segment (start 144.78 99.06) (end 145.88 99.06) (width 0.25) (layer B.Cu) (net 1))
 (segment (start 152.265001 104.640001) (end 152.265001 105.664999) (width 0.25) (layer B.Cu) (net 1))
 (segment (start 145.955001 99.135001) (end 145.955001 102.775001) (width 0.25) (layer B.Cu) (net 1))
 (segment (start 152.43 106.202) (end 152.43 106.68) (width 0.25) (layer B.Cu) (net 1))
 (segment (start 145.955001 102.775001) (end 146.594998 103.414998) (width 0.25) (layer B.Cu) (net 1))
 (segment (start 151.039998 103.414998) (end 152.265001 104.640001) (width 0.25) (layer B.Cu) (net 1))
 (segment (start 146.594998 103.414998) (end 151.039998 103.414998) (width 0.25) (layer B.Cu) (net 1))
 (segment (start 157.48 105.342081) (end 157.48 104.14) (width 0.25) (layer F.Cu) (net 10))
 (segment (start 157.48 105.47) (end 157.48 105.342081) (width 0.25) (layer F.Cu) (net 10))
 (segment (start 155.855 107.095) (end 157.48 105.47) (width 0.25) (layer F.Cu) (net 10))
 (segment (start 154.73 107.095) (end 155.855 107.095) (width 0.25) (layer F.Cu) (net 10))
 (segment (start 156.718 103.162998) (end 156.718 102.362) (width 0.25) (layer F.Cu) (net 14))
 (segment (start 156.718 102.362) (end 157.48 101.6) (width 0.25) (layer F.Cu) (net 14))
 (segment (start 156.304999 103.575999) (end 156.718 103.162998) (width 0.25) (layer F.Cu) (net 14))
 (segment (start 154.73 104.495) (end 155.765002 104.495) (width 0.25) (layer F.Cu) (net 14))
 (segment (start 156.304999 103.955003) (end 156.304999 103.575999) (width 0.25) (layer F.Cu) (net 14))
 (segment (start 155.765002 104.495) (end 156.304999 103.955003) (width 0.25) (layer F.Cu) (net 14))
 (segment (start 152.457685 103.124) (end 151.892 103.124) (width 0.25) (layer B.Cu) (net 11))
 (segment (start 154.88701 100.694675) (end 152.457685 103.124) (width 0.25) (layer B.Cu) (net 11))
 (segment (start 154.037 98.298) (end 154.88701 99.14801) (width 0.25) (layer B.Cu) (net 11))
 (segment (start 154.73 106.445) (end 153.605 106.445) (width 0.25) (layer F.Cu) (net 11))
 (via (at 151.892 103.124) (size 0.8) (drill 0.4) (layers F.Cu B.Cu) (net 11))
 (segment (start 154.88701 99.14801) (end 154.88701 100.694675) (width 0.25) (layer B.Cu) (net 11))
 (segment (start 153.605 106.445) (end 152.330989 105.170989) (width 0.25) (layer F.Cu) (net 11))
 (segment (start 152.330989 105.170989) (end 152.330989 103.562989) (width 0.25) (layer F.Cu) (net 11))
 (segment (start 152.330989 103.562989) (end 152.291999 103.523999) (width 0.25) (layer F.Cu) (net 11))
 (segment (start 152.291999 103.523999) (end 151.892 103.124) (width 0.25) (layer F.Cu) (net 11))
 (via (at 152.166724 102.162464) (size 0.8) (drill 0.4) (layers F.Cu B.Cu) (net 12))
 (segment (start 154.73 105.795) (end 153.605 105.795) (width 0.25) (layer F.Cu) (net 12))
 (segment (start 152.781 104.971) (end 152.781 102.77674) (width 0.25) (layer F.Cu) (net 12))
 (segment (start 154.037 100.076) (end 154.037 100.651) (width 0.25) (layer B.Cu) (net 12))
 (segment (start 152.566723 102.562463) (end 152.166724 102.162464) (width 0.25) (layer F.Cu) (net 12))
 (segment (start 153.605 105.795) (end 152.781 104.971) (width 0.25) (layer F.Cu) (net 12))
 (segment (start 152.781 102.77674) (end 152.566723 102.562463) (width 0.25) (layer F.Cu) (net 12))
 (segment (start 154.037 100.651) (end 152.525536 102.162464) (width 0.25) (layer B.Cu) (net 12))
 (segment (start 152.525536 102.162464) (end 152.166724 102.162464) (width 0.25) (layer B.Cu) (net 12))
 (segment (start 148.352 104.14) (end 148.717 104.505) (width 0.25) (layer B.Cu) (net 8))
 (segment (start 144.78 104.14) (end 148.352 104.14) (width 0.25) (layer B.Cu) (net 8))
 (segment (start 143.669999 97.884999) (end 143.51 98.044998) (width 0.25) (layer B.Cu) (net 9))
 (segment (start 147.129999 97.884999) (end 143.669999 97.884999) (width 0.25) (layer B.Cu) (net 9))
 (segment (start 148.717 98.822) (end 148.067 98.822) (width 0.25) (layer B.Cu) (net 9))
 (segment (start 148.067 98.822) (end 147.129999 97.884999) (width 0.25) (layer B.Cu) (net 9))
 (segment (start 143.51 100.33) (end 144.78 101.6) (width 0.25) (layer B.Cu) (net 9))
 (segment (start 143.51 98.044998) (end 143.51 100.33) (width 0.25) (layer B.Cu) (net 9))
 (segment (start 147.53 99.295) (end 148.655 99.295) (width 0.25) (layer F.Cu) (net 3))
 (segment (start 150.781339 105.885661) (end 150.876 105.791) (width 0.25) (layer F.Cu) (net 3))
 (segment (start 148.655 99.295) (end 149.642999 100.282999) (width 0.25) (layer F.Cu) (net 3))
 (segment (start 150.015339 105.885661) (end 150.781339 105.885661) (width 0.25) (layer F.Cu) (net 3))
 (segment (start 149.638339 104.812659) (end 149.638339 105.508661) (width 0.25) (layer F.Cu) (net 3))
 (segment (start 149.642999 100.282999) (end 149.642999 104.807999) (width 0.25) (layer F.Cu) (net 3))
 (segment (start 149.638339 105.508661) (end 150.015339 105.885661) (width 0.25) (layer F.Cu) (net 3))
 (segment (start 149.642999 104.807999) (end 149.638339 104.812659) (width 0.25) (layer F.Cu) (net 3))
 (via (at 151.44794 105.032635) (size 0.8) (drill 0.4) (layers F.Cu B.Cu) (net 3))
 (segment (start 150.876 105.791) (end 151.44794 105.21906) (width 0.25) (layer F.Cu) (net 3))
 (segment (start 151.44794 105.21906) (end 151.44794 105.032635) (width 0.25) (layer F.Cu) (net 3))
 (segment (start 151.78 105.364695) (end 151.78 106.68) (width 0.25) (layer B.Cu) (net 3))
 (segment (start 151.44794 105.032635) (end 151.78 105.364695) (width 0.25) (layer B.Cu) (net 3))
 (via (at 150.36334 105.16066) (size 0.8) (drill 0.4) (layers F.Cu B.Cu) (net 4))
 (segment (start 150.55066 105.16066) (end 150.36334 105.16066) (width 0.25) (layer B.Cu) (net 4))
 (segment (start 150.767999 104.756001) (end 150.763339 104.760661) (width 0.25) (layer F.Cu) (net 4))
 (segment (start 147.53 98.645) (end 148.655 98.645) (width 0.25) (layer F.Cu) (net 4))
 (segment (start 148.655 98.645) (end 150.767999 100.757999) (width 0.25) (layer F.Cu) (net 4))
 (segment (start 150.763339 104.760661) (end 150.36334 105.16066) (width 0.25) (layer F.Cu) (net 4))
 (segment (start 151.13 105.74) (end 150.55066 105.16066) (width 0.25) (layer B.Cu) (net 4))
 (segment (start 150.767999 100.757999) (end 150.767999 104.756001) (width 0.25) (layer F.Cu) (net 4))
 (segment (start 151.13 106.68) (end 151.13 105.74) (width 0.25) (layer B.Cu) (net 4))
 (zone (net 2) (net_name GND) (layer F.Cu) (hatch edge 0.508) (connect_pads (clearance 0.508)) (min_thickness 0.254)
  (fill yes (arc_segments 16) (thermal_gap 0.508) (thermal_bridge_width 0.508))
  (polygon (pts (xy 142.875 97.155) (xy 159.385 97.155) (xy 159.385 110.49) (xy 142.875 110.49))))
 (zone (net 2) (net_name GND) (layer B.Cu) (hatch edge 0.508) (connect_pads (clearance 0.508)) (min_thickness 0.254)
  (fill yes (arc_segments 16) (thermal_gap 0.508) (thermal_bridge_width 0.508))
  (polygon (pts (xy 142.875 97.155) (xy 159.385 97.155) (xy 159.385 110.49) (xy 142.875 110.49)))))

